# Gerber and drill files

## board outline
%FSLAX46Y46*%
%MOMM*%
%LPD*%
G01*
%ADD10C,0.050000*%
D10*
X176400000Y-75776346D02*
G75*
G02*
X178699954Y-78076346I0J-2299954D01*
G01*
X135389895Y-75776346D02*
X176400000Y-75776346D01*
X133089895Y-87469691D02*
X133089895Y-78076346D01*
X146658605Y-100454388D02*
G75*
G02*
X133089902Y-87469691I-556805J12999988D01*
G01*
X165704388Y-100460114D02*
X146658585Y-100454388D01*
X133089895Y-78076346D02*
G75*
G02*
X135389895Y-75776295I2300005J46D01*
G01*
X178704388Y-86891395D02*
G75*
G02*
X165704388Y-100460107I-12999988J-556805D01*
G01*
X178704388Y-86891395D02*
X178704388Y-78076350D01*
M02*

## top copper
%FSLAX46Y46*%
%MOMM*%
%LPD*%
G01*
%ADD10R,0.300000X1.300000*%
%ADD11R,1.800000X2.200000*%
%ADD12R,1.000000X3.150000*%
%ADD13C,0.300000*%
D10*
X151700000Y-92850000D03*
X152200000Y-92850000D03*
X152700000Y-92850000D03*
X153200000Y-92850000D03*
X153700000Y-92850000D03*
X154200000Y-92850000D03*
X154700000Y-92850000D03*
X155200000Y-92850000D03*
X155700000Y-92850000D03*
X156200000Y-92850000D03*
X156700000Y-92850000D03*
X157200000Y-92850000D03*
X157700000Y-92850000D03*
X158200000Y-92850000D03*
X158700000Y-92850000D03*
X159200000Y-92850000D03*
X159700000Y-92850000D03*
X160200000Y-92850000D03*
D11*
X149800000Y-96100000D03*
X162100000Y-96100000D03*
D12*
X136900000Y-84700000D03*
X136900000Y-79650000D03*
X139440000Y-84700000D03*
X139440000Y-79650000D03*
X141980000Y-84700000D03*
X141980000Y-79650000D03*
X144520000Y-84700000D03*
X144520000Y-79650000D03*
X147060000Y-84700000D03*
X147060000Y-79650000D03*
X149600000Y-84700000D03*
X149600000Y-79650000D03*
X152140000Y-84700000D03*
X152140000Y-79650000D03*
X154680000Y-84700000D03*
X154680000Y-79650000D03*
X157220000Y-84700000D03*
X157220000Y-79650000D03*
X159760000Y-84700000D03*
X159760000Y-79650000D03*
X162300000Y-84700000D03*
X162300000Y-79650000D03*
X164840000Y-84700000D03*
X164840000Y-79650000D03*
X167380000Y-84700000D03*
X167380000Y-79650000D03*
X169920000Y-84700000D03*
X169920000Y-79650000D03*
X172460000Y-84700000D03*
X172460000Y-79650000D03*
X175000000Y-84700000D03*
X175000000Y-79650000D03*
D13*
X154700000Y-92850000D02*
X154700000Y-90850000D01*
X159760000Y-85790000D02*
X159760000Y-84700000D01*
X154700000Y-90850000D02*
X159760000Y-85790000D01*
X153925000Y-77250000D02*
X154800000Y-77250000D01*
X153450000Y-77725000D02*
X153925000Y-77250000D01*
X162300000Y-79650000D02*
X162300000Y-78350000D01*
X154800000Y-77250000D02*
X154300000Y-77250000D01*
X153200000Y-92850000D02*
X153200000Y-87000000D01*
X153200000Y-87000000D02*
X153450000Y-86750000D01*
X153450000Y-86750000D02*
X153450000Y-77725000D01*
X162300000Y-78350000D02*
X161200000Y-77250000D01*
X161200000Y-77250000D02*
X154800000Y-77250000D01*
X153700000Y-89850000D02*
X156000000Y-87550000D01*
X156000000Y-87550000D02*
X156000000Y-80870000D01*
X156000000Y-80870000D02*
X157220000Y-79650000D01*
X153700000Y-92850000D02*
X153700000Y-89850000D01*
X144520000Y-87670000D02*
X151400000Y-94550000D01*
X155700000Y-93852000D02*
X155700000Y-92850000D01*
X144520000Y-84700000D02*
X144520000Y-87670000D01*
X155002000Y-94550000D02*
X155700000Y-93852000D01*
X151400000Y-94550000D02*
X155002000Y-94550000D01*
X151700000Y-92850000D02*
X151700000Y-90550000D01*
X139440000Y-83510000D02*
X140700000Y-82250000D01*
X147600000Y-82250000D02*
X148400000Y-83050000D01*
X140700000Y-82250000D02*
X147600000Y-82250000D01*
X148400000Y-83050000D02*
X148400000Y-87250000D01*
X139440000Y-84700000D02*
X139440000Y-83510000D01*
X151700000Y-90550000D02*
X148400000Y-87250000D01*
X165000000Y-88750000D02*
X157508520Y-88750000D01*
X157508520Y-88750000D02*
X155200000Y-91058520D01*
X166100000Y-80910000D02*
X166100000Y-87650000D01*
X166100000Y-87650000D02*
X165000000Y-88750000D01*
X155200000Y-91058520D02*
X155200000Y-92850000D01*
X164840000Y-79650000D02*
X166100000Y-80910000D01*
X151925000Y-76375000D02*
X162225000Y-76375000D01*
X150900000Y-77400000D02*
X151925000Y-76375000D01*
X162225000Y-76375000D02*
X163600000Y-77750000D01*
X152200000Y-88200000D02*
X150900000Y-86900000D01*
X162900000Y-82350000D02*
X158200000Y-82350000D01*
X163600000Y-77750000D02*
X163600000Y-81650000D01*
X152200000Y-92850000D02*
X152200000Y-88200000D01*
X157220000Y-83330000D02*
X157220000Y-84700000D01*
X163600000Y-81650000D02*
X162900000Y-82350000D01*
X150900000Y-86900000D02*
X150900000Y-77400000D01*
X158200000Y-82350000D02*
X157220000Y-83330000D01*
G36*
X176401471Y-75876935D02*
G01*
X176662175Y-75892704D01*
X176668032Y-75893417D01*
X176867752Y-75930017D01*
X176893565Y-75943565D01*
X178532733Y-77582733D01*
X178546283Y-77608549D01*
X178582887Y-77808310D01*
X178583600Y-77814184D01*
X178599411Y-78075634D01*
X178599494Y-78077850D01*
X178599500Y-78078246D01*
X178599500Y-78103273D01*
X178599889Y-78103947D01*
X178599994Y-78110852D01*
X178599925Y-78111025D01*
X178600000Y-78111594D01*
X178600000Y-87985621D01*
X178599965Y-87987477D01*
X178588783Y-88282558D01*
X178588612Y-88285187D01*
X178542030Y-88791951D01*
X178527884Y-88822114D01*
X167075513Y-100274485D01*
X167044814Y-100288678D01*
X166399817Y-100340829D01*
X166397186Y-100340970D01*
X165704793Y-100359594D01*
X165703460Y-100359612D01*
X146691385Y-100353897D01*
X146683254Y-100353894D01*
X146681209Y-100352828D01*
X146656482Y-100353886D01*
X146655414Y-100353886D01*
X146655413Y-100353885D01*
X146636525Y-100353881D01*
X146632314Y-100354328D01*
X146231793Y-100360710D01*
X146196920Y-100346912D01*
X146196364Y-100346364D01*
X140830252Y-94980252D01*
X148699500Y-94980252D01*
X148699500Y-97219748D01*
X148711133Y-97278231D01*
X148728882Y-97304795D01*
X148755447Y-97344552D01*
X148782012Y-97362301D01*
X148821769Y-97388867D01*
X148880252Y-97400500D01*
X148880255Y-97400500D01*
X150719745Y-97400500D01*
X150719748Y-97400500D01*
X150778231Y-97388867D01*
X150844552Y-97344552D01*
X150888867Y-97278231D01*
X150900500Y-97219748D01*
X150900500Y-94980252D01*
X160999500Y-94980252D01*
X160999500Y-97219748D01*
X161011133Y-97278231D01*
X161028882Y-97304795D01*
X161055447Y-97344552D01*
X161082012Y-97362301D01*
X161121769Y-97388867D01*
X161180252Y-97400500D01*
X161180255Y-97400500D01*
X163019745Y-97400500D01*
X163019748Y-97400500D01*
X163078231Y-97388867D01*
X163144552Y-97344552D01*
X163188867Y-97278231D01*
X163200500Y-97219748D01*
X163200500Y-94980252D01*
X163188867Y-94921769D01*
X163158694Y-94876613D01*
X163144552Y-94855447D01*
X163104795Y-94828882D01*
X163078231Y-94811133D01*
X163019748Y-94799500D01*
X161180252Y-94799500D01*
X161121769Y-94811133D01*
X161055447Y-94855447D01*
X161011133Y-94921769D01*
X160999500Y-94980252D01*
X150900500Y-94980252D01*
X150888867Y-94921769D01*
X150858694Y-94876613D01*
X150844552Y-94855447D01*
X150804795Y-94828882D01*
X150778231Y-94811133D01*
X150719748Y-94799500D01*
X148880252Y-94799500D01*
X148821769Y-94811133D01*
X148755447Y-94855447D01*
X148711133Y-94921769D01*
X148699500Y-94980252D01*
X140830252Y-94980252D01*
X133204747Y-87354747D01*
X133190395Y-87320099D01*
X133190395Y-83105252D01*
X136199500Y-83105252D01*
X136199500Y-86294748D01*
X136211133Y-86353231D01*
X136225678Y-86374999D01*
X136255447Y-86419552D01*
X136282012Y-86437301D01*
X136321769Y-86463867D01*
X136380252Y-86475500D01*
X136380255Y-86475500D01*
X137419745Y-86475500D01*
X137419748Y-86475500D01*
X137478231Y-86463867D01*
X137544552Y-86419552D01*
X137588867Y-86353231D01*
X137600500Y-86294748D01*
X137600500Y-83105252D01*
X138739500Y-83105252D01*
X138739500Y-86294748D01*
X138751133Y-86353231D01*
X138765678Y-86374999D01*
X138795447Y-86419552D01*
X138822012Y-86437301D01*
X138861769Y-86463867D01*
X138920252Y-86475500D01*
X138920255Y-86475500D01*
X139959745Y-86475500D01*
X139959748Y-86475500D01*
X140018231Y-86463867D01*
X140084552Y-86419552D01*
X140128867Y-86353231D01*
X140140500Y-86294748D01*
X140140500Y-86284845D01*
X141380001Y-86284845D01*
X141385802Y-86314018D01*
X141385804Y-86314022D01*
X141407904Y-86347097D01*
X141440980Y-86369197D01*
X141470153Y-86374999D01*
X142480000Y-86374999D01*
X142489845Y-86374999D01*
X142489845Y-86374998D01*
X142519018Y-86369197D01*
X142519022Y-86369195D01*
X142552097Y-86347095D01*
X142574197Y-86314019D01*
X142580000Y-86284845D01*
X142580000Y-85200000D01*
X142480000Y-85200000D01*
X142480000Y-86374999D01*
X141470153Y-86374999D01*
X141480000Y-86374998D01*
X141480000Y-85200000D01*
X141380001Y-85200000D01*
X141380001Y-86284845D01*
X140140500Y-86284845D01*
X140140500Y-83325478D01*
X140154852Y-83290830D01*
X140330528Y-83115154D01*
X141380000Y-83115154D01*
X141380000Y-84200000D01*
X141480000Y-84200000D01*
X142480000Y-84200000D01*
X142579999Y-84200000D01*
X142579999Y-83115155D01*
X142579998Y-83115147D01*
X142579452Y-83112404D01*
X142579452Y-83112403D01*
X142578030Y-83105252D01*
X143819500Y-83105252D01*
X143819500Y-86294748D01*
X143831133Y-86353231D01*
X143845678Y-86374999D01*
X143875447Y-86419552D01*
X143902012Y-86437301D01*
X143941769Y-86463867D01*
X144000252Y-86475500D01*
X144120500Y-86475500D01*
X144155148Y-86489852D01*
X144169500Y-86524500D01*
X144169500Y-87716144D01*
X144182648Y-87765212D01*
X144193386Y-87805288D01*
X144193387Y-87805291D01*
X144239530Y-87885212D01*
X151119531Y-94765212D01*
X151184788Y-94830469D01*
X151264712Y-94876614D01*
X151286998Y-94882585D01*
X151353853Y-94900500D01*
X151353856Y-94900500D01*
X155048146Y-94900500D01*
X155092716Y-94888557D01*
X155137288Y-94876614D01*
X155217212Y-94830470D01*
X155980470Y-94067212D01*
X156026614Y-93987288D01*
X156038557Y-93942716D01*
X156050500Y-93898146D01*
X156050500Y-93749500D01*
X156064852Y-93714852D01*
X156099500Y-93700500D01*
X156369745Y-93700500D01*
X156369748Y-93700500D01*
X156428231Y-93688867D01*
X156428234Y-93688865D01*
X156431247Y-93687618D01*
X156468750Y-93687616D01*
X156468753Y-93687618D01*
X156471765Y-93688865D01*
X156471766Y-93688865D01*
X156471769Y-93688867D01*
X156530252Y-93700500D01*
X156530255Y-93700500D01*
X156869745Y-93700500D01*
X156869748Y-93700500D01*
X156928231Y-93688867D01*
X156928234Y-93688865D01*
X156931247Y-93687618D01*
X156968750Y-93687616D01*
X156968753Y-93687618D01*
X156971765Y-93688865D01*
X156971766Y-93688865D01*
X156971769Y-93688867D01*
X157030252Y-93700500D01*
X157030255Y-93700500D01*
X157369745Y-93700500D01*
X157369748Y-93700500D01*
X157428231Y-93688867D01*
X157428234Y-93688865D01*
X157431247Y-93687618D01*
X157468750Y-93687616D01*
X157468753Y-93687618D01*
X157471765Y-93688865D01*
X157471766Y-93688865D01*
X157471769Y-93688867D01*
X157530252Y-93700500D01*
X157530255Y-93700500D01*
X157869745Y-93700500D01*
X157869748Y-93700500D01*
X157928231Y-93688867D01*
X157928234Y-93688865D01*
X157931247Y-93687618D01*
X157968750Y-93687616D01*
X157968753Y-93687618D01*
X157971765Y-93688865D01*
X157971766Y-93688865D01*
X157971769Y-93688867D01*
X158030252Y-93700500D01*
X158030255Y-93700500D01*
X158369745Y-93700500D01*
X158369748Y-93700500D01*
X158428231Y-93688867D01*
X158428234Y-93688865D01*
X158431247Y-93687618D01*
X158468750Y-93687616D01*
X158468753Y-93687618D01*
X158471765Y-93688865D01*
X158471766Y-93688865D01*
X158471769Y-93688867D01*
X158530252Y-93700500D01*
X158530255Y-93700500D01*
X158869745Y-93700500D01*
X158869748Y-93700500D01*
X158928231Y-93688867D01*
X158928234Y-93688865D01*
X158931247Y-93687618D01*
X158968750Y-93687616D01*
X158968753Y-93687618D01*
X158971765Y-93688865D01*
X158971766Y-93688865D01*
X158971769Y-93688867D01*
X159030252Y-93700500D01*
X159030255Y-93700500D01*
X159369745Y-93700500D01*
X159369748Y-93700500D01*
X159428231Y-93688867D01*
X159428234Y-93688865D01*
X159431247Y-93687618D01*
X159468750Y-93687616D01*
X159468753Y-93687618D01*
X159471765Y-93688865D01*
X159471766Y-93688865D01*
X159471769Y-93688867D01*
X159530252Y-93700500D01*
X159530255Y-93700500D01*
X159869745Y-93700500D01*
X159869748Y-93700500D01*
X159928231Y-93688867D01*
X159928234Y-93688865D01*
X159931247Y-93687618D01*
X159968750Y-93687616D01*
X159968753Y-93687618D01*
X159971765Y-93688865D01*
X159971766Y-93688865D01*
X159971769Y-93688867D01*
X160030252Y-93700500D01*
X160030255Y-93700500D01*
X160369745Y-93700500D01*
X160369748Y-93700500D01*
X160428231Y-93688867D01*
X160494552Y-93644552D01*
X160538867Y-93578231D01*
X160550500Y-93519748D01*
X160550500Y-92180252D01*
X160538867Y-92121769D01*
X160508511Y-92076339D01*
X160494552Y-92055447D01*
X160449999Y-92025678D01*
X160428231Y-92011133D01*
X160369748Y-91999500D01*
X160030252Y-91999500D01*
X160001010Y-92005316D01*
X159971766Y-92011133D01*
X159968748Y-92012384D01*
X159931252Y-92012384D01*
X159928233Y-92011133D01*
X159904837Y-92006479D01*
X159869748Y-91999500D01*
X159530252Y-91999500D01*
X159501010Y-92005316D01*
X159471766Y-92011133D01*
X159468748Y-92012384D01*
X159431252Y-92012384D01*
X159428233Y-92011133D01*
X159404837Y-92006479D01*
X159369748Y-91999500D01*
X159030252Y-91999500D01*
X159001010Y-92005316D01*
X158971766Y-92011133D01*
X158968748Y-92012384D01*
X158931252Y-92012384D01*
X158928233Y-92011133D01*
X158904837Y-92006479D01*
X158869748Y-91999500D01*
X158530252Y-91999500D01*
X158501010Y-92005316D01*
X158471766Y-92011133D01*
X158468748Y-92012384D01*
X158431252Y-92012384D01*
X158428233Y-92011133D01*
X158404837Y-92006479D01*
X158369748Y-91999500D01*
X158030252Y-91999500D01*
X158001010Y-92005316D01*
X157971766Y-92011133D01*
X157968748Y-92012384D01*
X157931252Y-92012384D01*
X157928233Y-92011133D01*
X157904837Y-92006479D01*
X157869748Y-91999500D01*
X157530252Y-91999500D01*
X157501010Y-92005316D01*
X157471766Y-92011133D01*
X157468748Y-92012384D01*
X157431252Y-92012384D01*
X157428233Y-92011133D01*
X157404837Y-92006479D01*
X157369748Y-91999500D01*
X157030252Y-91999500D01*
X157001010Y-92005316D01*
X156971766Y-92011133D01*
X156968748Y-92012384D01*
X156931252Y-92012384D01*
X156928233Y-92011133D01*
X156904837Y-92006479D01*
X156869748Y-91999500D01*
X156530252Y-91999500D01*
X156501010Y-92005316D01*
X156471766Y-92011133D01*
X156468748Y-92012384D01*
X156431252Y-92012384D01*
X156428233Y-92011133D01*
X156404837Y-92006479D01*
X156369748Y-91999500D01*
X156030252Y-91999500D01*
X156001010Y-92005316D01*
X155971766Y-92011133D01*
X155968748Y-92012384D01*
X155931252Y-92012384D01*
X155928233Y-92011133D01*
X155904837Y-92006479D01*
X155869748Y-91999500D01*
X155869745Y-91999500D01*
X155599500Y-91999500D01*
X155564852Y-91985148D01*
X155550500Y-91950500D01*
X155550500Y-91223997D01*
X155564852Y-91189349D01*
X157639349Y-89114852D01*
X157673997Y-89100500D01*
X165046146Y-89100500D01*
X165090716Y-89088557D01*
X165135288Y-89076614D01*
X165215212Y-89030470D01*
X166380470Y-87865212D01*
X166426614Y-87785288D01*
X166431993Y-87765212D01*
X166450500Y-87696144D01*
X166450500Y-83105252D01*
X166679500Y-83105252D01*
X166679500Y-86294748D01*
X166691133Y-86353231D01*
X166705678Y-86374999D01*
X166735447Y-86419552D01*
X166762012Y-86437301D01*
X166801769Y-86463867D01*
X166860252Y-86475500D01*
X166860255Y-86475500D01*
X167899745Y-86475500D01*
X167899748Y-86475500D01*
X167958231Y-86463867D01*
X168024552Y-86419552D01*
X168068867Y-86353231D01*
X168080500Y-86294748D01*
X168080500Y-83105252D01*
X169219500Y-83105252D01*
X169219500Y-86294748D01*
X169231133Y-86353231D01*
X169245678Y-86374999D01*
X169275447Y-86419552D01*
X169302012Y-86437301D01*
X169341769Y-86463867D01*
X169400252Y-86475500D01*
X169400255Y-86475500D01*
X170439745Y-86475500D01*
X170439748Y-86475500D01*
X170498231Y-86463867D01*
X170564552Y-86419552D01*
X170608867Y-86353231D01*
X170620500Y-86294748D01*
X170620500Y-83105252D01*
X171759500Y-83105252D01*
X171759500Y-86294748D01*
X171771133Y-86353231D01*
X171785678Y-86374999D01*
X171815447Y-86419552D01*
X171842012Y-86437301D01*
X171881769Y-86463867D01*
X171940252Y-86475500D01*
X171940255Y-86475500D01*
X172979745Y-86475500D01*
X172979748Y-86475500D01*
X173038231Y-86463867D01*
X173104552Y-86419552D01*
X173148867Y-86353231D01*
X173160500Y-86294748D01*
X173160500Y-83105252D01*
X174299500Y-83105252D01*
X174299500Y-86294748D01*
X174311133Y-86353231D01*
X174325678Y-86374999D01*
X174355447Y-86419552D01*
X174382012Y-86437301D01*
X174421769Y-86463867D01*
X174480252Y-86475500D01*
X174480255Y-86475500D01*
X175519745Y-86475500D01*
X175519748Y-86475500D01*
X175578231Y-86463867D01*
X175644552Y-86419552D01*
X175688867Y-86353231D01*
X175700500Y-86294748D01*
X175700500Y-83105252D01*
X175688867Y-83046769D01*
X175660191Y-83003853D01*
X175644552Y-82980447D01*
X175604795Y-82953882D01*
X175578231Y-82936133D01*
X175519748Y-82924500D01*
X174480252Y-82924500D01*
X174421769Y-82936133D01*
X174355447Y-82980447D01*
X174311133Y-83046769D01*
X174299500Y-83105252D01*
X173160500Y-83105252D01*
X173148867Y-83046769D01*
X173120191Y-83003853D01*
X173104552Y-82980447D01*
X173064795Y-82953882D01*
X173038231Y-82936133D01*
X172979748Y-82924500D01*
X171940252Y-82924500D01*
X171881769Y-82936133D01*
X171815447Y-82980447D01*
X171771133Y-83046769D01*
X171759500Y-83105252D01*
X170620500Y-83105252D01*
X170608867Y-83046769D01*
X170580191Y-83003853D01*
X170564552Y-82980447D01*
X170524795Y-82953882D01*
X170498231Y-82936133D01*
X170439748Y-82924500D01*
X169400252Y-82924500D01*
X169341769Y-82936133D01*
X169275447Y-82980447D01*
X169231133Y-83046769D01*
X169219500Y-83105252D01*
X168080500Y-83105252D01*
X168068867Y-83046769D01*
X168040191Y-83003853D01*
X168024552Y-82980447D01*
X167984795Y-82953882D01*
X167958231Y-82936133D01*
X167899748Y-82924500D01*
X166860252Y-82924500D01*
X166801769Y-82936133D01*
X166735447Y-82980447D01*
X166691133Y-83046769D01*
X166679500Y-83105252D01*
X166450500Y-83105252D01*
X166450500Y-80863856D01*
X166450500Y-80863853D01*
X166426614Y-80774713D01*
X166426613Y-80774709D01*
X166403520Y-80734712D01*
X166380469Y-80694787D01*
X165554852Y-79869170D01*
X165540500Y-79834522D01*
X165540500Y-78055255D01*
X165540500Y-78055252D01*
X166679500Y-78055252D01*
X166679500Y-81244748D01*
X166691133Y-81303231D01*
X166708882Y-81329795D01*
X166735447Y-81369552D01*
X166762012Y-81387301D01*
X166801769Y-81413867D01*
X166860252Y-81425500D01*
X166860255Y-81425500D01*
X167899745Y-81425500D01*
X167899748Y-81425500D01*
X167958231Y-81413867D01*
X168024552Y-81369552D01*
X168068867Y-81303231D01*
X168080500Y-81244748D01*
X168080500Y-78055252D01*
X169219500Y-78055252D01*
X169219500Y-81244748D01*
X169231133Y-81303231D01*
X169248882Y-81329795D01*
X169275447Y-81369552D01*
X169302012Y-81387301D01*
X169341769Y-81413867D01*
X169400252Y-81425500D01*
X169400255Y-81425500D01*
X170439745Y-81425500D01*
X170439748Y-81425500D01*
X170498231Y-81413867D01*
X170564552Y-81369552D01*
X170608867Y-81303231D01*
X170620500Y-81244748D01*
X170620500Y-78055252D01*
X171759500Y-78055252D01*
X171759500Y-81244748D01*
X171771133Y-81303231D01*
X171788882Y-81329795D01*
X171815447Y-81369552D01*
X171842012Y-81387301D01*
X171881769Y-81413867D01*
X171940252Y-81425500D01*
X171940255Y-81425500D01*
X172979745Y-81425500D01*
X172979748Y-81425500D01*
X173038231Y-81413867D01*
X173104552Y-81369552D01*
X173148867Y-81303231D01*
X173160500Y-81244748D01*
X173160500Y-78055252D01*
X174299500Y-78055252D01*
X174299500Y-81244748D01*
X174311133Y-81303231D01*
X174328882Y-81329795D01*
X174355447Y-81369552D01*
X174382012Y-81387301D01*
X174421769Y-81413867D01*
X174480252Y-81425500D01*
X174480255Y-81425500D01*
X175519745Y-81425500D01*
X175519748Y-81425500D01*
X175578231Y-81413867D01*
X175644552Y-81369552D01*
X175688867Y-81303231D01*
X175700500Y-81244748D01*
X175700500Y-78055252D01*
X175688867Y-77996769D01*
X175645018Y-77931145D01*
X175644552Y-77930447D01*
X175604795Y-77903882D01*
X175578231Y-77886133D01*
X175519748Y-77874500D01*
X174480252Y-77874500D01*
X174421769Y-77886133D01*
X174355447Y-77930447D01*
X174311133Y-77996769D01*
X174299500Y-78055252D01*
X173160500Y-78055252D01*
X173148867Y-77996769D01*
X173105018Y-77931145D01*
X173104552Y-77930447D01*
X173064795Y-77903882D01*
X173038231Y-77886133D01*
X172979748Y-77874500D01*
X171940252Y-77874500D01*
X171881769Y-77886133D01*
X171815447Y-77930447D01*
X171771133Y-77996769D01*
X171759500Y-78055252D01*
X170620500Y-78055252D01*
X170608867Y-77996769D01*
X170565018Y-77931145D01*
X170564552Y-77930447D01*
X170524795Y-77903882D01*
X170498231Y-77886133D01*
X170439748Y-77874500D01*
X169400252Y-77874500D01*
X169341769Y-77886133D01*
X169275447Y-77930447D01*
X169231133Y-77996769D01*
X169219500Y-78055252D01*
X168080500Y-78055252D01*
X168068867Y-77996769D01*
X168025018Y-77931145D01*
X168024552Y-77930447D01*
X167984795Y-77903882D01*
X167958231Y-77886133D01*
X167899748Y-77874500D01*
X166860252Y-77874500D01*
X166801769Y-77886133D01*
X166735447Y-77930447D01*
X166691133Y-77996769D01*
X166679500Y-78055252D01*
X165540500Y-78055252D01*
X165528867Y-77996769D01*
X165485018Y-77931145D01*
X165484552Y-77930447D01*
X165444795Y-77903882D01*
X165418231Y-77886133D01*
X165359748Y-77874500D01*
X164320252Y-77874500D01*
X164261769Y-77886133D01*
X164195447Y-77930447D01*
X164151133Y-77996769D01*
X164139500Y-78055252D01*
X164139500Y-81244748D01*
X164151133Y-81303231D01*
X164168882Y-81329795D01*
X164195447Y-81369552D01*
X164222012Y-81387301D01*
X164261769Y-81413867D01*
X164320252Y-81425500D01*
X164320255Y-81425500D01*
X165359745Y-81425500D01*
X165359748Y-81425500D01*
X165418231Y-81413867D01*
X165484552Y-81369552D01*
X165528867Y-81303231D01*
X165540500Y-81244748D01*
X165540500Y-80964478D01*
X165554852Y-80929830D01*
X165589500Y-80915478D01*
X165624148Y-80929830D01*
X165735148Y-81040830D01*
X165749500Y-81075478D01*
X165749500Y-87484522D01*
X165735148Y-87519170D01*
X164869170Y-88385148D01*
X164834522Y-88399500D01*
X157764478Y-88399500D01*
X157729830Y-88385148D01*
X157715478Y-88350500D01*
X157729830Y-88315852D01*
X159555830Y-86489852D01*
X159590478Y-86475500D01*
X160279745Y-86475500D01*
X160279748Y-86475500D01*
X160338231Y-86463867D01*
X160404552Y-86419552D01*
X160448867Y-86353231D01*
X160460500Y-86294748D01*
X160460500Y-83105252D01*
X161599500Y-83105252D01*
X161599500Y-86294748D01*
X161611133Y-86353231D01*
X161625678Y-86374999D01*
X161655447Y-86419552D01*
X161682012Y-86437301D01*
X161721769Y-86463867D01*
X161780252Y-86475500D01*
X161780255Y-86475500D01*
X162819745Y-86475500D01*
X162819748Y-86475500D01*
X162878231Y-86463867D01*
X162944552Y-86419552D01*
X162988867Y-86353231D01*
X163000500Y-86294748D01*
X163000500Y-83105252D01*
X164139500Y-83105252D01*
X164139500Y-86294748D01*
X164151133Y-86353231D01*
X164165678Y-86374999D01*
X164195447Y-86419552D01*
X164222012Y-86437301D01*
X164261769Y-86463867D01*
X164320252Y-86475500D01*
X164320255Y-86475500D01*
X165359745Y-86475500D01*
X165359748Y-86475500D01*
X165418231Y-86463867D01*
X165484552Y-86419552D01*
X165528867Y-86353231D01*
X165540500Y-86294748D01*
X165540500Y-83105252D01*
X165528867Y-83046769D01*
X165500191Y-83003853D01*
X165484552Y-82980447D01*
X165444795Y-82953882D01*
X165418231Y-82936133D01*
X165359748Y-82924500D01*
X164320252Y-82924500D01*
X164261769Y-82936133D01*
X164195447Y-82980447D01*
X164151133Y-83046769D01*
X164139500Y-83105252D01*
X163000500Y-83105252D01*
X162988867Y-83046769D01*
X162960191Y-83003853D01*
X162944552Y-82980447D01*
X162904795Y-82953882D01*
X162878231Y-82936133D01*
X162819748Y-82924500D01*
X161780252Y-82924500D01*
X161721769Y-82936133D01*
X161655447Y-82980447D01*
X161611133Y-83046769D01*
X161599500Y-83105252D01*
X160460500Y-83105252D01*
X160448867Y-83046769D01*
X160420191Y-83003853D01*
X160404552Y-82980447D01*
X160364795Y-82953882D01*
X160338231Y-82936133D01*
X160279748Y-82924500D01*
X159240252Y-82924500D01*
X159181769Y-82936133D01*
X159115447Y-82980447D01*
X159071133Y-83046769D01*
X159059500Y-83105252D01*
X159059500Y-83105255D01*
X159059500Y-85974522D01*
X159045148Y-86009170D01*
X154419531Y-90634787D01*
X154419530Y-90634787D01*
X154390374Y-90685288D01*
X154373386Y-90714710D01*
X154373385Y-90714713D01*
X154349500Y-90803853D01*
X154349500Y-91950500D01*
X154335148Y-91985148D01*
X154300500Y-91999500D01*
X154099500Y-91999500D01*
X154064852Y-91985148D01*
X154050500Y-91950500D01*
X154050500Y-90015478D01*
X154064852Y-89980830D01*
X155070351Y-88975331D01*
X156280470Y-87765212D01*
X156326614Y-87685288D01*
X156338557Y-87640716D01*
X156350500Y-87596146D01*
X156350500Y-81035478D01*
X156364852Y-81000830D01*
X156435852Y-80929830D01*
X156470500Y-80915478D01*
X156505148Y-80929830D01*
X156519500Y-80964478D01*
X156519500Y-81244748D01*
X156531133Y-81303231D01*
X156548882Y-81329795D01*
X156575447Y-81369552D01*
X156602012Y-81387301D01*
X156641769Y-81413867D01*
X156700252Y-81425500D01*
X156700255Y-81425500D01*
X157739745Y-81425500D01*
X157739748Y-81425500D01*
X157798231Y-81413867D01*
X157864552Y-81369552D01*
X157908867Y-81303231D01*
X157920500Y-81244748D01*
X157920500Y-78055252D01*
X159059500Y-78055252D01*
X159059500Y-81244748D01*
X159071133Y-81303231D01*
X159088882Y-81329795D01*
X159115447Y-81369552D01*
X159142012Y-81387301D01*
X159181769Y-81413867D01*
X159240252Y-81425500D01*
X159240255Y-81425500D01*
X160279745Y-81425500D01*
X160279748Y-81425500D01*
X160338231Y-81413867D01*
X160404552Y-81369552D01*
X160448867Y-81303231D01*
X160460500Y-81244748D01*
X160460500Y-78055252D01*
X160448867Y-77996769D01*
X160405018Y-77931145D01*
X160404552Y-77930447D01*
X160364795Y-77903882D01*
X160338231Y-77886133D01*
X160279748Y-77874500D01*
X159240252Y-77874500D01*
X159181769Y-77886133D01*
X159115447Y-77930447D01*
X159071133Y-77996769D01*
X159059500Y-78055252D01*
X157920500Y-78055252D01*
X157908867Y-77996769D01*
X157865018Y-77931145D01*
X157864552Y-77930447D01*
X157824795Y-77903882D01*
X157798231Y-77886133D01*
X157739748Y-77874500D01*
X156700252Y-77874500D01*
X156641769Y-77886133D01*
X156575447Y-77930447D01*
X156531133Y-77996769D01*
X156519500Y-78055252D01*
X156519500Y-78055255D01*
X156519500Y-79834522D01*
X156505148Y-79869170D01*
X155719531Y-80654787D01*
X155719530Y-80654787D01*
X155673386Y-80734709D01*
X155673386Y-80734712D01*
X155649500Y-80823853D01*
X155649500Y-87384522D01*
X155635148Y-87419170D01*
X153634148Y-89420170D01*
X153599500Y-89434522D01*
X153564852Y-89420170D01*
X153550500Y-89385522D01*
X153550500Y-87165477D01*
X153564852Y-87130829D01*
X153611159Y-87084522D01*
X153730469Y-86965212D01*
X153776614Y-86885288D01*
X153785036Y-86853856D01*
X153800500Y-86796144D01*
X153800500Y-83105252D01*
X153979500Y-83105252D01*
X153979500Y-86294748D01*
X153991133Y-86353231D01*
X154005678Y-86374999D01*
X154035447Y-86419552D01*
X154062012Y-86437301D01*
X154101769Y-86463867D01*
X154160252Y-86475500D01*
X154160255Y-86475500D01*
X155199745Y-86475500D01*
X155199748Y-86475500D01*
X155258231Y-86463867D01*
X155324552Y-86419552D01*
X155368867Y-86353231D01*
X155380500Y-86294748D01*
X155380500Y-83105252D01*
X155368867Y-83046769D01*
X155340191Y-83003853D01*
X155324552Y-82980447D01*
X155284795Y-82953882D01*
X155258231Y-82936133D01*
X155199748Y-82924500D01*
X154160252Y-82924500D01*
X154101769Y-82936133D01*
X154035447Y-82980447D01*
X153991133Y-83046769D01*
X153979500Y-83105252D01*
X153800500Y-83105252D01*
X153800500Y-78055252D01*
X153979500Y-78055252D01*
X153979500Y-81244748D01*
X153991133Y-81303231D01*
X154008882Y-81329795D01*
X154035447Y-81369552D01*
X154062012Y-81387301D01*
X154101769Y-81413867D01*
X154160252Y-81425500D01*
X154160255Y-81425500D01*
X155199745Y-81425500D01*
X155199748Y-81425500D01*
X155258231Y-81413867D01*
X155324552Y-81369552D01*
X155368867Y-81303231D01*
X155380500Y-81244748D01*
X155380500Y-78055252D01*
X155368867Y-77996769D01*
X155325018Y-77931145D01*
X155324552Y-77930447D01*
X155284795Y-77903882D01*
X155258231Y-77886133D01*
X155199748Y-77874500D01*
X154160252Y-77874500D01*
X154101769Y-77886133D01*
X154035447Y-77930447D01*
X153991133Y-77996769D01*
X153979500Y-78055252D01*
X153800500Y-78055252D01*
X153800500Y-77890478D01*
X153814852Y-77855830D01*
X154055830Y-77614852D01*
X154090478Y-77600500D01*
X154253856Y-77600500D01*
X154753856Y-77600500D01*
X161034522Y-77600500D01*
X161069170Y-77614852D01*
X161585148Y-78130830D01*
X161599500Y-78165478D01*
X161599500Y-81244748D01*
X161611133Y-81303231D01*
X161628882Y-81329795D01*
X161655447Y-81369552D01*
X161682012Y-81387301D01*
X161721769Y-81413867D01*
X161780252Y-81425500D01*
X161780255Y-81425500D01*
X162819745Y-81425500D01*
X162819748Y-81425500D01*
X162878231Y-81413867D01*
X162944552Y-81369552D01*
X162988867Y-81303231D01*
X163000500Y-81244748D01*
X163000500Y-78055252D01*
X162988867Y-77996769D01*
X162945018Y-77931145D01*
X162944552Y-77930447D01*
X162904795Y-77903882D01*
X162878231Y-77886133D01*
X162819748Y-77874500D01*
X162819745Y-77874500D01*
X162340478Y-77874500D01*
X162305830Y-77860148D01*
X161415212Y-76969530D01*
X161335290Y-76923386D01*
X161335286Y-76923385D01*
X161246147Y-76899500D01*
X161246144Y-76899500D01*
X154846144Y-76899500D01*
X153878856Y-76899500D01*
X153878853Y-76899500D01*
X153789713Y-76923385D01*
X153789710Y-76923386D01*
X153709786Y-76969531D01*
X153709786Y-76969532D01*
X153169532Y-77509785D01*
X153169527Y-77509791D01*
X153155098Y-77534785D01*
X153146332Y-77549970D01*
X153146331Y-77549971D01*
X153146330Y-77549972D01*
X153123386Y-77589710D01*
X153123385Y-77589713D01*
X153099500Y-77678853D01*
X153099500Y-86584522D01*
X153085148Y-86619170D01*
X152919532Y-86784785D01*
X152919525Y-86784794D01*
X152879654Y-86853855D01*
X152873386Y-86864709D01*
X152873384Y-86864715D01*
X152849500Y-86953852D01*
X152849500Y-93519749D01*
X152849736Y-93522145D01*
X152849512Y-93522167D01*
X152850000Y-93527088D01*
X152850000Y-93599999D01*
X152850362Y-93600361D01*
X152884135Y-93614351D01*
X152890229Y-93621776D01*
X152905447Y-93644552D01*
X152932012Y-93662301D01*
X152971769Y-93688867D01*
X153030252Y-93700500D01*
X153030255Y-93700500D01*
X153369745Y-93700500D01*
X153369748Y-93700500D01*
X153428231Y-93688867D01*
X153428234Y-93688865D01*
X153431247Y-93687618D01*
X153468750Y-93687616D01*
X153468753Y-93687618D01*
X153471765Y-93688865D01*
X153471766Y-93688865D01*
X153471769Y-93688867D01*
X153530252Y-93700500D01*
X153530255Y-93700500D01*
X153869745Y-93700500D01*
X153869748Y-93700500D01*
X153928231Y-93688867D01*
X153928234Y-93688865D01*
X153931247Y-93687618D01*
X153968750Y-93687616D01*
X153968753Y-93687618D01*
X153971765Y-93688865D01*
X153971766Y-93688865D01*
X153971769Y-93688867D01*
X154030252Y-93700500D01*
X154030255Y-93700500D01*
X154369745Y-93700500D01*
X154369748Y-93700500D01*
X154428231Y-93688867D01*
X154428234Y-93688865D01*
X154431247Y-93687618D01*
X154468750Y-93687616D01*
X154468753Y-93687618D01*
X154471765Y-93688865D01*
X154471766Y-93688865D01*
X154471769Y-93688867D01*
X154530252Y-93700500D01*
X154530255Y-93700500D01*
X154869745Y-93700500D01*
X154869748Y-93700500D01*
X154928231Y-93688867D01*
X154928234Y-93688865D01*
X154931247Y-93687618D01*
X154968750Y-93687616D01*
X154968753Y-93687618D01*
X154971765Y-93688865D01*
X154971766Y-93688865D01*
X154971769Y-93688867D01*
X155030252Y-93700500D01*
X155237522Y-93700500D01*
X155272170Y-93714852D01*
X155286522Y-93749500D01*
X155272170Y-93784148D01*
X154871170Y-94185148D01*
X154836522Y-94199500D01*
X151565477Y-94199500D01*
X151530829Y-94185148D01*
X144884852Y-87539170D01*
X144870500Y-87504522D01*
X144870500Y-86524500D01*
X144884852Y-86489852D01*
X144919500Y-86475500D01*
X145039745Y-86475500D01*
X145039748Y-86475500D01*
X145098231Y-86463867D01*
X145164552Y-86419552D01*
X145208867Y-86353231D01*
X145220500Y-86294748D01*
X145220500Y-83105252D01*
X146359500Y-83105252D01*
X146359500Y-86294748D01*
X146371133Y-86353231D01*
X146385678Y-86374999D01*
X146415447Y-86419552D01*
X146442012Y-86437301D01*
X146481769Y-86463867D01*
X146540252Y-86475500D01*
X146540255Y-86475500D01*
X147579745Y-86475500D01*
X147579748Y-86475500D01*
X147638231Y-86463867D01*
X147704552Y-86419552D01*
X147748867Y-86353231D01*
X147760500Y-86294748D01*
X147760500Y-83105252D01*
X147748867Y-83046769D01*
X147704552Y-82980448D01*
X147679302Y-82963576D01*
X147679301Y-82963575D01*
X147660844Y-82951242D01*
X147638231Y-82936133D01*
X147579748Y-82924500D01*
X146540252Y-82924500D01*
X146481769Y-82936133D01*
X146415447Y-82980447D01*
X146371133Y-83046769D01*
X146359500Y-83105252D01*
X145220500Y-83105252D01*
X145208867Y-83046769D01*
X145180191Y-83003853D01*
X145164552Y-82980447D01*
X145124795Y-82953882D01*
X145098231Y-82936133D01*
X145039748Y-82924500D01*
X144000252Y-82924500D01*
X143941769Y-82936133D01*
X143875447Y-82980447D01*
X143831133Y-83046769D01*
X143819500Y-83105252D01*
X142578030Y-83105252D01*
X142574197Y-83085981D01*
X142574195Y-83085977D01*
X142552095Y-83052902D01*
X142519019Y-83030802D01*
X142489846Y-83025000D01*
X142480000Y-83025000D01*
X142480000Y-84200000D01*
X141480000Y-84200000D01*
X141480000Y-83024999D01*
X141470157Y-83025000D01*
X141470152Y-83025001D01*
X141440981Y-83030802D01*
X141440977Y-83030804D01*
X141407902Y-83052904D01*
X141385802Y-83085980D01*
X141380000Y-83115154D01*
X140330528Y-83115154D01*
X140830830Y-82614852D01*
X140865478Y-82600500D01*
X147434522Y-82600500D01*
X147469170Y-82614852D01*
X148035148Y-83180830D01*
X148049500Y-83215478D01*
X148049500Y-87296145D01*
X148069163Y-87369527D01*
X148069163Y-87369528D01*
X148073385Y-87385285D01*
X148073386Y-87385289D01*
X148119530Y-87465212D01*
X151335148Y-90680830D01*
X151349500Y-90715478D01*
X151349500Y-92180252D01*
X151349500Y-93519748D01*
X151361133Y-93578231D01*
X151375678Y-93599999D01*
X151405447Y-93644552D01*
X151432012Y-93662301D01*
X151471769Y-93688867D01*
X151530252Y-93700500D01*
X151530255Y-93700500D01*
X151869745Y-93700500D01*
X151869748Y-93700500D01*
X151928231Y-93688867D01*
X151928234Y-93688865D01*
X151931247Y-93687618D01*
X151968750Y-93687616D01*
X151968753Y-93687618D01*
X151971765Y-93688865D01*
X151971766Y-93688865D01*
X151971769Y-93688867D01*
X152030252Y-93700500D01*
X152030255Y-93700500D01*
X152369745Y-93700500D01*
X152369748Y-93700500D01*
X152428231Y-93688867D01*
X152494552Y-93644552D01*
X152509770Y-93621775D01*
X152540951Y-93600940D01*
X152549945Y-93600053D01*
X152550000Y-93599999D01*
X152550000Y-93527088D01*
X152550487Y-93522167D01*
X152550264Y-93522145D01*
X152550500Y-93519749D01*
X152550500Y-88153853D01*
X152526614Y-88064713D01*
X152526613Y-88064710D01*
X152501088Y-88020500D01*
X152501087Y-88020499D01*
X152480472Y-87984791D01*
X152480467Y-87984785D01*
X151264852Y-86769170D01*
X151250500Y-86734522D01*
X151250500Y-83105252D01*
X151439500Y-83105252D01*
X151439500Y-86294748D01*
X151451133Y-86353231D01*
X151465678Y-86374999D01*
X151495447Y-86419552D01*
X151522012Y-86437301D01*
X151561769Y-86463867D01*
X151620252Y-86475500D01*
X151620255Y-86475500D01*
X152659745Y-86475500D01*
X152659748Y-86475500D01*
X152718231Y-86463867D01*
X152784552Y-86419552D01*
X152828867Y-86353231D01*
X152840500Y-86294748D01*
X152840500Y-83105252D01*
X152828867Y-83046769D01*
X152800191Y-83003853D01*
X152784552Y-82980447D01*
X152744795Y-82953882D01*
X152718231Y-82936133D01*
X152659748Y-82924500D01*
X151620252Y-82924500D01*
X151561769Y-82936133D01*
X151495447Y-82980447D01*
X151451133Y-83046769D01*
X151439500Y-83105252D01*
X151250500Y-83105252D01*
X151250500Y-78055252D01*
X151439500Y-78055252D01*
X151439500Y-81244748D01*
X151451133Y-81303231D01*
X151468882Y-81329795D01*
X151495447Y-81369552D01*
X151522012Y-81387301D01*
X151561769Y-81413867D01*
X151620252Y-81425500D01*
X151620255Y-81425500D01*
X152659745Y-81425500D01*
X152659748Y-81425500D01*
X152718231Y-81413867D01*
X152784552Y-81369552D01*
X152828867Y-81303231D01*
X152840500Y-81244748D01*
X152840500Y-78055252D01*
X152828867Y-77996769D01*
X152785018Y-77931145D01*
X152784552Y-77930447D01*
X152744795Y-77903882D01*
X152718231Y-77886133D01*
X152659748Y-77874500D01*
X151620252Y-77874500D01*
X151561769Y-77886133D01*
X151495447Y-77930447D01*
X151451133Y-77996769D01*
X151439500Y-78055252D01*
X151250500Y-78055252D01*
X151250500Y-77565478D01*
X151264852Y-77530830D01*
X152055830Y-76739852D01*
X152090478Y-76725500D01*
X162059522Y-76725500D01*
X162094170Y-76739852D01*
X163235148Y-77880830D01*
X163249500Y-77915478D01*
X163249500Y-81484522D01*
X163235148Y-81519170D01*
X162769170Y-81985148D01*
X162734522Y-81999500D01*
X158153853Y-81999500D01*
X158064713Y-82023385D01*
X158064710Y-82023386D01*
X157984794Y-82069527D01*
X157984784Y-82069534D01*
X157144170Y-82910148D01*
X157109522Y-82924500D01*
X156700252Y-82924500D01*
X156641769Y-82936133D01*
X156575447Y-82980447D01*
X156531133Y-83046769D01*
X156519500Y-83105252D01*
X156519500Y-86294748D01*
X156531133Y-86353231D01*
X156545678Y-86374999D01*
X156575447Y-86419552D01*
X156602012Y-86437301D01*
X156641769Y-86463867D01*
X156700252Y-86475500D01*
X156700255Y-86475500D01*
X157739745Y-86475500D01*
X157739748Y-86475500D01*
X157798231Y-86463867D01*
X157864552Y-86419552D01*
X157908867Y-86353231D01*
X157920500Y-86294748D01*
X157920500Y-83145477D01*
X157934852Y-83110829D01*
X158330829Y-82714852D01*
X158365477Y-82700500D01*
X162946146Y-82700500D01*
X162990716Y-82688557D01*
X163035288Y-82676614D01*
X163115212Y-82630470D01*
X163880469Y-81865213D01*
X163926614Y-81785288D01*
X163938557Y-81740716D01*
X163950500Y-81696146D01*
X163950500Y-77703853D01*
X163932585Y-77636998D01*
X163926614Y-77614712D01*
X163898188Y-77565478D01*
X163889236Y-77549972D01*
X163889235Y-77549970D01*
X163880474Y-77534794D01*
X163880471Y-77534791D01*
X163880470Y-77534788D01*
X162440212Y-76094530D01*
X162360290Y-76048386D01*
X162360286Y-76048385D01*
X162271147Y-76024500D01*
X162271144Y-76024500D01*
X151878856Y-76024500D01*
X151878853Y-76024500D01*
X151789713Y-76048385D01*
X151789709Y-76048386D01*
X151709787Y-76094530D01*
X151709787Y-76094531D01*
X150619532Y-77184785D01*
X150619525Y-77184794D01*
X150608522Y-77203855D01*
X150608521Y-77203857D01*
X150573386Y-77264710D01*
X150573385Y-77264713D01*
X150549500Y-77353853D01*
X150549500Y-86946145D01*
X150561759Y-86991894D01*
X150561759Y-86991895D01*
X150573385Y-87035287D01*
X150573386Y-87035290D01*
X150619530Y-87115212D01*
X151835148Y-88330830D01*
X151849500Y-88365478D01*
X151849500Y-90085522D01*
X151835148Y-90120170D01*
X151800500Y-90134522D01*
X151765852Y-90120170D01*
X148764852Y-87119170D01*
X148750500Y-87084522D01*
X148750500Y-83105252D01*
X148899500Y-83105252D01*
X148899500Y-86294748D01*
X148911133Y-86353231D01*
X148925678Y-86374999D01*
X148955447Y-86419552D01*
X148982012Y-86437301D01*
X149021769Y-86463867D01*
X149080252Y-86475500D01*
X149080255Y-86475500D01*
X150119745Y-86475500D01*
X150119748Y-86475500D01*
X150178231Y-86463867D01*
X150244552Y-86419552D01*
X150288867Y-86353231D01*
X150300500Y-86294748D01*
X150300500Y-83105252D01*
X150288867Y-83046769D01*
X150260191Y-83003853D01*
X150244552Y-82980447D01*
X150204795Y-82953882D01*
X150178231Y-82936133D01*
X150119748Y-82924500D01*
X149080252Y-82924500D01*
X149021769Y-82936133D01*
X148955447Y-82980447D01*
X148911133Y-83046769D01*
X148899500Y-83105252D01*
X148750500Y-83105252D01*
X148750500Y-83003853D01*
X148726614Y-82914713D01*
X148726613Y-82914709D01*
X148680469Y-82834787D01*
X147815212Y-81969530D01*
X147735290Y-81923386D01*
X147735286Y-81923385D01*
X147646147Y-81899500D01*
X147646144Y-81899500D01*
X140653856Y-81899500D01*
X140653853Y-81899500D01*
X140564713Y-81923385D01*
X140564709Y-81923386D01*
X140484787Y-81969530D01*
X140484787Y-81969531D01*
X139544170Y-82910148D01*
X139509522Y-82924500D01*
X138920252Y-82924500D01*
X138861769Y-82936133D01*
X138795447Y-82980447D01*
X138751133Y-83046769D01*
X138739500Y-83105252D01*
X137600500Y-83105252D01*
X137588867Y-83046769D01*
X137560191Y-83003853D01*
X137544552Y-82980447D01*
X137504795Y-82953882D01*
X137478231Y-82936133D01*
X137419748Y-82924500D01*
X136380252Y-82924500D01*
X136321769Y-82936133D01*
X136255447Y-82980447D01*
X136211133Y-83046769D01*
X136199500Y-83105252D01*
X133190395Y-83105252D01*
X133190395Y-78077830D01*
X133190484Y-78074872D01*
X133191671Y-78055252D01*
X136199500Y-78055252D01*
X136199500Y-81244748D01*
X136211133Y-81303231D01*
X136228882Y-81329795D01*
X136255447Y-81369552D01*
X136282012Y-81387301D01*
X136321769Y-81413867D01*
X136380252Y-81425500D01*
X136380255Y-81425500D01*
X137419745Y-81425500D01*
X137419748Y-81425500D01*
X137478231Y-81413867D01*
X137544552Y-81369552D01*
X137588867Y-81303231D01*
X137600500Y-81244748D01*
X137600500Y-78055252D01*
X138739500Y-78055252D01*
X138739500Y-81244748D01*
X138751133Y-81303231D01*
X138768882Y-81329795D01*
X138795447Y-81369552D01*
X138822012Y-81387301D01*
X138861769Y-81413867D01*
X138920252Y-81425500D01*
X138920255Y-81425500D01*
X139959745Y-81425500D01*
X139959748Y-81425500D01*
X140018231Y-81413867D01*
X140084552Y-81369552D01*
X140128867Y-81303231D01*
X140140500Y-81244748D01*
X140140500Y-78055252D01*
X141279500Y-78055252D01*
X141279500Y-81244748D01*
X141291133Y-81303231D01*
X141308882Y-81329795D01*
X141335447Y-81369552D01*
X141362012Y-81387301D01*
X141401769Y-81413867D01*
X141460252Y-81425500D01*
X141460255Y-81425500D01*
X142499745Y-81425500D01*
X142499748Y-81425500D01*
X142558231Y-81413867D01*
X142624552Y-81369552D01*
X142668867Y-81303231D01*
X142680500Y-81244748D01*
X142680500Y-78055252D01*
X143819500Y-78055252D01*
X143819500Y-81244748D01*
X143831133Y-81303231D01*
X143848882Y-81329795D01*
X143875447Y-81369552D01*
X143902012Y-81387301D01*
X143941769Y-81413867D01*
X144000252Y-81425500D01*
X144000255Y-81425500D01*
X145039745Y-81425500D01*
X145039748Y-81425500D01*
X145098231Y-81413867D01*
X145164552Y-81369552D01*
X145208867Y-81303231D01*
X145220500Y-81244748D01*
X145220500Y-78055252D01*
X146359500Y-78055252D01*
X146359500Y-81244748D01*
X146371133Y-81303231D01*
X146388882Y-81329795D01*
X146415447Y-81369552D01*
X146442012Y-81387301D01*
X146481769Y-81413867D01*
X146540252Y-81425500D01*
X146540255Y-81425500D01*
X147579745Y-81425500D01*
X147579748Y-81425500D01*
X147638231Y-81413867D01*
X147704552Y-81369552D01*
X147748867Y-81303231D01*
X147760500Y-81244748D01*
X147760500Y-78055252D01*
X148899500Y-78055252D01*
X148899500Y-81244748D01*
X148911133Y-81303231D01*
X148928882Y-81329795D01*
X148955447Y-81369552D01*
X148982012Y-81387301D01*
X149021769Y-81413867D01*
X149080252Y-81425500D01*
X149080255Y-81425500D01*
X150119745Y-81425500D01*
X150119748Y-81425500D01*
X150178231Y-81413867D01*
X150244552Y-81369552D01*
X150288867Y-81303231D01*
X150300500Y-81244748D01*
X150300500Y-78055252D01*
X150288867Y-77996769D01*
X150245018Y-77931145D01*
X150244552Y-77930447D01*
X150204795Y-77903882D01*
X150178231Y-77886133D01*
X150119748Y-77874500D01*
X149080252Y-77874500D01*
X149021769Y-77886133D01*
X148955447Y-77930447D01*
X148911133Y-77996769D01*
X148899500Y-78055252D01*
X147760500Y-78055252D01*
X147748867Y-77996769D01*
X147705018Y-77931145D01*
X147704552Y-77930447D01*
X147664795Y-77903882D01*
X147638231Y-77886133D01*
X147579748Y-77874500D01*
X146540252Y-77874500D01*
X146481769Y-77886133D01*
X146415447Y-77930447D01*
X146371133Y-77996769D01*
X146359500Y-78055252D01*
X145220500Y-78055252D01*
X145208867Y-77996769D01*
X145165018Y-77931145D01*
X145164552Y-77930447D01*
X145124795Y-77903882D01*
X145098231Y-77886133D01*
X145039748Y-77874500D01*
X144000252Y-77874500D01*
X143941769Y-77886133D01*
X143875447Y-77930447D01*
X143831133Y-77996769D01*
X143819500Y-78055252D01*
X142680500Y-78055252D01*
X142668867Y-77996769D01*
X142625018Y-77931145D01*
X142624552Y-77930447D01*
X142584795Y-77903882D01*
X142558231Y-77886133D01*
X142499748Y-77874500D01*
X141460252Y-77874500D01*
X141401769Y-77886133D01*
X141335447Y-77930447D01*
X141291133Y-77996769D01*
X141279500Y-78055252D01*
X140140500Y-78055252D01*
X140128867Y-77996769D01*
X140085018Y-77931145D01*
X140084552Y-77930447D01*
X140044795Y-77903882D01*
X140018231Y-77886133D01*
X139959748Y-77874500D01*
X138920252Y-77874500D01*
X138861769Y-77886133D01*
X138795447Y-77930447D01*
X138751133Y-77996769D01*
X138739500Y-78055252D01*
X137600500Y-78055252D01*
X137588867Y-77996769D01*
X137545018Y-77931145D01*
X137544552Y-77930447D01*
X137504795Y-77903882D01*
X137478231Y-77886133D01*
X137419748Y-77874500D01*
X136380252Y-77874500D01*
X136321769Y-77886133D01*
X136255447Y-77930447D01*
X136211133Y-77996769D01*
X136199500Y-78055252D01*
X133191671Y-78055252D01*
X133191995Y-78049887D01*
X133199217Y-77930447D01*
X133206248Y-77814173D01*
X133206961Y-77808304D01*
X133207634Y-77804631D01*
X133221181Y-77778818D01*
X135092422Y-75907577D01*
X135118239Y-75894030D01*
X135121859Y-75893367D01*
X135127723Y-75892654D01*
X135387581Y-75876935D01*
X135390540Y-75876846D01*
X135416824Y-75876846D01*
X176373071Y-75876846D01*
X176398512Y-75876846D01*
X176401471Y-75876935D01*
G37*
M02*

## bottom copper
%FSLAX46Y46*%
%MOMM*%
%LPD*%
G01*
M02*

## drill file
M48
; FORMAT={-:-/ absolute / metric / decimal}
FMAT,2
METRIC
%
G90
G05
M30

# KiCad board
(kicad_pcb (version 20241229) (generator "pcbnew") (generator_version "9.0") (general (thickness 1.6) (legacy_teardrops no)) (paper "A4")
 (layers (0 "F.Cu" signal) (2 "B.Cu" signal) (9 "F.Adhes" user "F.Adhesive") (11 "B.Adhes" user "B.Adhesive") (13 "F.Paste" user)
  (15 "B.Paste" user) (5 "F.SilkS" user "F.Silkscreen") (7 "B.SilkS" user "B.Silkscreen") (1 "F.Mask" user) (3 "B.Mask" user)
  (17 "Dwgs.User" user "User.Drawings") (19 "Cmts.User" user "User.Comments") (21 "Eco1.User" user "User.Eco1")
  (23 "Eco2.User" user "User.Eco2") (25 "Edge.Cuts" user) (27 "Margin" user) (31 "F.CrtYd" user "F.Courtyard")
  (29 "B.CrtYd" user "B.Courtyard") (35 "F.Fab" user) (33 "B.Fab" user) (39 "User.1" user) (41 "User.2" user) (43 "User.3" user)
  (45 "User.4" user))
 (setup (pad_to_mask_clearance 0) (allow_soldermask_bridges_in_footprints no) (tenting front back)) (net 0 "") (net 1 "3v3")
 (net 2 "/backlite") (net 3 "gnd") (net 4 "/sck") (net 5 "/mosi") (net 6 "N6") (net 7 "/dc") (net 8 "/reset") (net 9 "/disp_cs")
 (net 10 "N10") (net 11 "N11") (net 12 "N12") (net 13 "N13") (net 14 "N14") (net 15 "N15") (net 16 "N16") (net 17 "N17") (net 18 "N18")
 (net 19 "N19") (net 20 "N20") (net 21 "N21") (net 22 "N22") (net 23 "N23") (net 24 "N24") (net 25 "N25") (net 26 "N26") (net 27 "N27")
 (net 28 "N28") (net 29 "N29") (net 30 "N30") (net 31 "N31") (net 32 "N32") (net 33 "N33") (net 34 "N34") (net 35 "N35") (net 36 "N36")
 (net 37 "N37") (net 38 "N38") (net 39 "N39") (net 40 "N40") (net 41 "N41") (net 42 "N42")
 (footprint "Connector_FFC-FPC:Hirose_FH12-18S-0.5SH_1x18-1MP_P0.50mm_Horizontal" (layer "F.Cu") (at 155.95 94.7)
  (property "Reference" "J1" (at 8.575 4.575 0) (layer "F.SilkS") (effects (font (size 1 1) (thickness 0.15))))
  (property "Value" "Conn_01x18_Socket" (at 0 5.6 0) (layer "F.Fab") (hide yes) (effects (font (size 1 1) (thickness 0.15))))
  (pad "1" smd rect (at -4.25 -1.85) (size 0.3 1.3) (layers "F.Cu" "F.Mask" "F.Paste") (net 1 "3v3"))
  (pad "2" smd rect (at -3.75 -1.85) (size 0.3 1.3) (layers "F.Cu" "F.Mask" "F.Paste") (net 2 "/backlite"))
  (pad "3" smd rect (at -3.25 -1.85) (size 0.3 1.3) (layers "F.Cu" "F.Mask" "F.Paste") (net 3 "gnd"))
  (pad "4" smd rect (at -2.75 -1.85) (size 0.3 1.3) (layers "F.Cu" "F.Mask" "F.Paste") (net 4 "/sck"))
  (pad "5" smd rect (at -2.25 -1.85) (size 0.3 1.3) (layers "F.Cu" "F.Mask" "F.Paste") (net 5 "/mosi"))
  (pad "6" smd rect (at -1.75 -1.85) (size 0.3 1.3) (layers "F.Cu" "F.Mask" "F.Paste") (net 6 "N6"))
  (pad "7" smd rect (at -1.25 -1.85) (size 0.3 1.3) (layers "F.Cu" "F.Mask" "F.Paste") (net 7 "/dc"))
  (pad "8" smd rect (at -0.75 -1.85) (size 0.3 1.3) (layers "F.Cu" "F.Mask" "F.Paste") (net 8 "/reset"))
  (pad "9" smd rect (at -0.25 -1.85) (size 0.3 1.3) (layers "F.Cu" "F.Mask" "F.Paste") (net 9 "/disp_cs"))
  (pad "10" smd rect (at 0.25 -1.85) (size 0.3 1.3) (layers "F.Cu" "F.Mask" "F.Paste") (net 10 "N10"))
  (pad "11" smd rect (at 0.75 -1.85) (size 0.3 1.3) (layers "F.Cu" "F.Mask" "F.Paste") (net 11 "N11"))
  (pad "12" smd rect (at 1.25 -1.85) (size 0.3 1.3) (layers "F.Cu" "F.Mask" "F.Paste") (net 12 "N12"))
  (pad "13" smd rect (at 1.75 -1.85) (size 0.3 1.3) (layers "F.Cu" "F.Mask" "F.Paste") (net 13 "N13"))
  (pad "14" smd rect (at 2.25 -1.85) (size 0.3 1.3) (layers "F.Cu" "F.Mask" "F.Paste") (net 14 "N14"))
  (pad "15" smd rect (at 2.75 -1.85) (size 0.3 1.3) (layers "F.Cu" "F.Mask" "F.Paste") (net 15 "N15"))
  (pad "16" smd rect (at 3.25 -1.85) (size 0.3 1.3) (layers "F.Cu" "F.Mask" "F.Paste") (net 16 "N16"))
  (pad "17" smd rect (at 3.75 -1.85) (size 0.3 1.3) (layers "F.Cu" "F.Mask" "F.Paste") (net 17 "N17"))
  (pad "18" smd rect (at 4.25 -1.85) (size 0.3 1.3) (layers "F.Cu" "F.Mask" "F.Paste") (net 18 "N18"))
  (pad "MP" smd rect (at -6.15 1.4) (size 1.8 2.2) (layers "F.Cu" "F.Mask" "F.Paste"))
  (pad "MP" smd rect (at 6.15 1.4) (size 1.8 2.2) (layers "F.Cu" "F.Mask" "F.Paste")))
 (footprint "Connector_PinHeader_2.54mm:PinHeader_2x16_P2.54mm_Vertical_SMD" (layer "F.Cu") (at 155.95 82.175 90)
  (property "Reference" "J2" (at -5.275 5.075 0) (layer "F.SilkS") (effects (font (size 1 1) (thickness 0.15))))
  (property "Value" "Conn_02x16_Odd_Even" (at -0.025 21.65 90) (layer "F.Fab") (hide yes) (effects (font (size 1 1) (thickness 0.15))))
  (pad "1" smd rect (at -2.525 -19.05 90) (size 3.15 1) (layers "F.Cu" "F.Mask" "F.Paste") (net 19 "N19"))
  (pad "2" smd rect (at 2.525 -19.05 90) (size 3.15 1) (layers "F.Cu" "F.Mask" "F.Paste") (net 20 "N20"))
  (pad "3" smd rect (at -2.525 -16.51 90) (size 3.15 1) (layers "F.Cu" "F.Mask" "F.Paste") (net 1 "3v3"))
  (pad "4" smd rect (at 2.525 -16.51 90) (size 3.15 1) (layers "F.Cu" "F.Mask" "F.Paste") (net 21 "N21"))
  (pad "5" smd rect (at -2.525 -13.97 90) (size 3.15 1) (layers "F.Cu" "F.Mask" "F.Paste") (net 3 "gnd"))
  (pad "6" smd rect (at 2.525 -13.97 90) (size 3.15 1) (layers "F.Cu" "F.Mask" "F.Paste") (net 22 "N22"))
  (pad "7" smd rect (at -2.525 -11.43 90) (size 3.15 1) (layers "F.Cu" "F.Mask" "F.Paste") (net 9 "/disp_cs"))
  (pad "8" smd rect (at 2.525 -11.43 90) (size 3.15 1) (layers "F.Cu" "F.Mask" "F.Paste") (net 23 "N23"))
  (pad "9" smd rect (at -2.525 -8.89 90) (size 3.15 1) (layers "F.Cu" "F.Mask" "F.Paste") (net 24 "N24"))
  (pad "10" smd rect (at 2.525 -8.89 90) (size 3.15 1) (layers "F.Cu" "F.Mask" "F.Paste") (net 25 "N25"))
  (pad "11" smd rect (at -2.525 -6.35 90) (size 3.15 1) (layers "F.Cu" "F.Mask" "F.Paste") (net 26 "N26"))
  (pad "12" smd rect (at 2.525 -6.35 90) (size 3.15 1) (layers "F.Cu" "F.Mask" "F.Paste") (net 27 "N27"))
  (pad "13" smd rect (at -2.525 -3.81 90) (size 3.15 1) (layers "F.Cu" "F.Mask" "F.Paste") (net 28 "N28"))
  (pad "14" smd rect (at 2.525 -3.81 90) (size 3.15 1) (layers "F.Cu" "F.Mask" "F.Paste") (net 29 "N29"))
  (pad "15" smd rect (at -2.525 -1.27 90) (size 3.15 1) (layers "F.Cu" "F.Mask" "F.Paste") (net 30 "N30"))
  (pad "16" smd rect (at 2.525 -1.27 90) (size 3.15 1) (layers "F.Cu" "F.Mask" "F.Paste") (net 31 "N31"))
  (pad "17" smd rect (at -2.525 1.27 90) (size 3.15 1) (layers "F.Cu" "F.Mask" "F.Paste") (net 2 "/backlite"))
  (pad "18" smd rect (at 2.525 1.27 90) (size 3.15 1) (layers "F.Cu" "F.Mask" "F.Paste") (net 5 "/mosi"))
  (pad "19" smd rect (at -2.525 3.81 90) (size 3.15 1) (layers "F.Cu" "F.Mask" "F.Paste") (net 7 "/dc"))
  (pad "20" smd rect (at 2.525 3.81 90) (size 3.15 1) (layers "F.Cu" "F.Mask" "F.Paste") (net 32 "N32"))
  (pad "21" smd rect (at -2.525 6.35 90) (size 3.15 1) (layers "F.Cu" "F.Mask" "F.Paste") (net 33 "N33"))
  (pad "22" smd rect (at 2.525 6.35 90) (size 3.15 1) (layers "F.Cu" "F.Mask" "F.Paste") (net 4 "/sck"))
  (pad "23" smd rect (at -2.525 8.89 90) (size 3.15 1) (layers "F.Cu" "F.Mask" "F.Paste") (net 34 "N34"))
  (pad "24" smd rect (at 2.525 8.89 90) (size 3.15 1) (layers "F.Cu" "F.Mask" "F.Paste") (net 8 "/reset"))
  (pad "25" smd rect (at -2.525 11.43 90) (size 3.15 1) (layers "F.Cu" "F.Mask" "F.Paste") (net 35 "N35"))
  (pad "26" smd rect (at 2.525 11.43 90) (size 3.15 1) (layers "F.Cu" "F.Mask" "F.Paste") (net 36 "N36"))
  (pad "27" smd rect (at -2.525 13.97 90) (size 3.15 1) (layers "F.Cu" "F.Mask" "F.Paste") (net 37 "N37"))
  (pad "28" smd rect (at 2.525 13.97 90) (size 3.15 1) (layers "F.Cu" "F.Mask" "F.Paste") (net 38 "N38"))
  (pad "29" smd rect (at -2.525 16.51 90) (size 3.15 1) (layers "F.Cu" "F.Mask" "F.Paste") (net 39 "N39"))
  (pad "30" smd rect (at 2.525 16.51 90) (size 3.15 1) (layers "F.Cu" "F.Mask" "F.Paste") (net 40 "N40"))
  (pad "31" smd rect (at -2.525 19.05 90) (size 3.15 1) (layers "F.Cu" "F.Mask" "F.Paste") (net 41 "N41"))
  (pad "32" smd rect (at 2.525 19.05 90) (size 3.15 1) (layers "F.Cu" "F.Mask" "F.Paste") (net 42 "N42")))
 (gr_arc (start 176.4 75.776346) (mid 178.026346 76.45) (end 178.7 78.076346) (stroke (width 0.05) (type default)) (layer "Edge.Cuts"))
 (gr_line (start 135.389895 75.776346) (end 176.4 75.776346) (stroke (width 0.05) (type default)) (layer "Edge.Cuts"))
 (gr_line (start 133.089895 87.469691) (end 133.089895 78.076346) (stroke (width 0.05) (type default)) (layer "Edge.Cuts"))
 (gr_arc (start 146.658605 100.454388) (mid 137.105527 96.855292) (end 133.089895 87.469691) (stroke (width 0.05) (type default))
  (layer "Edge.Cuts"))
 (gr_line (start 165.704388 100.460114) (end 146.658585 100.454388) (stroke (width 0.05) (type default)) (layer "Edge.Cuts"))
 (gr_arc (start 133.089895 78.076346) (mid 133.763549 76.45) (end 135.389895 75.776346) (stroke (width 0.05) (type default))
  (layer "Edge.Cuts"))
 (gr_arc (start 178.704388 86.891395) (mid 175.1 96.45) (end 165.704388 100.460114) (stroke (width 0.05) (type default)) (layer "Edge.Cuts"))
 (gr_line (start 178.704388 86.891395) (end 178.704388 78.07635) (stroke (width 0.05) (type default)) (layer "Edge.Cuts"))
 (segment (start 154.7 92.85) (end 154.7 90.85) (width 0.3) (layer "F.Cu") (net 7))
 (segment (start 159.76 85.79) (end 159.76 84.7) (width 0.3) (layer "F.Cu") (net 7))
 (segment (start 154.7 90.85) (end 159.76 85.79) (width 0.3) (layer "F.Cu") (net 7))
 (segment (start 153.925 77.25) (end 154.8 77.25) (width 0.3) (layer "F.Cu") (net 4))
 (segment (start 153.45 77.725) (end 153.925 77.25) (width 0.3) (layer "F.Cu") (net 4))
 (segment (start 162.3 79.65) (end 162.3 78.35) (width 0.3) (layer "F.Cu") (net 4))
 (segment (start 154.8 77.25) (end 154.3 77.25) (width 0.3) (layer "F.Cu") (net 4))
 (segment (start 153.2 92.85) (end 153.2 87) (width 0.3) (layer "F.Cu") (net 4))
 (segment (start 153.2 87) (end 153.45 86.75) (width 0.3) (layer "F.Cu") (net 4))
 (segment (start 153.45 86.75) (end 153.45 77.725) (width 0.3) (layer "F.Cu") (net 4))
 (segment (start 162.3 78.35) (end 161.2 77.25) (width 0.3) (layer "F.Cu") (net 4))
 (segment (start 161.2 77.25) (end 154.8 77.25) (width 0.3) (layer "F.Cu") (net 4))
 (segment (start 153.7 89.85) (end 156 87.55) (width 0.3) (layer "F.Cu") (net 5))
 (segment (start 156 87.55) (end 156 80.87) (width 0.3) (layer "F.Cu") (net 5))
 (segment (start 156 80.87) (end 157.22 79.65) (width 0.3) (layer "F.Cu") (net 5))
 (segment (start 153.7 92.85) (end 153.7 89.85) (width 0.3) (layer "F.Cu") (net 5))
 (segment (start 144.52 87.67) (end 151.4 94.55) (width 0.3) (layer "F.Cu") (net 9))
 (segment (start 155.7 93.852) (end 155.7 92.85) (width 0.3) (layer "F.Cu") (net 9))
 (segment (start 144.52 84.7) (end 144.52 87.67) (width 0.3) (layer "F.Cu") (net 9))
 (segment (start 155.002 94.55) (end 155.7 93.852) (width 0.3) (layer "F.Cu") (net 9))
 (segment (start 151.4 94.55) (end 155.002 94.55) (width 0.3) (layer "F.Cu") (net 9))
 (segment (start 151.7 92.85) (end 151.7 90.55) (width 0.3) (layer "F.Cu") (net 1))
 (segment (start 139.44 83.51) (end 140.7 82.25) (width 0.3) (layer "F.Cu") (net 1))
 (segment (start 147.6 82.25) (end 148.4 83.05) (width 0.3) (layer "F.Cu") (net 1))
 (segment (start 140.7 82.25) (end 147.6 82.25) (width 0.3) (layer "F.Cu") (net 1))
 (segment (start 148.4 83.05) (end 148.4 87.25) (width 0.3) (layer "F.Cu") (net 1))
 (segment (start 139.44 84.7) (end 139.44 83.51) (width 0.3) (layer "F.Cu") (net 1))
 (segment (start 151.7 90.55) (end 148.4 87.25) (width 0.3) (layer "F.Cu") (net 1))
 (segment (start 165 88.75) (end 157.50852 88.75) (width 0.3) (layer "F.Cu") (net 8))
 (segment (start 157.50852 88.75) (end 155.2 91.05852) (width 0.3) (layer "F.Cu") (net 8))
 (segment (start 166.1 80.91) (end 166.1 87.65) (width 0.3) (layer "F.Cu") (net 8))
 (segment (start 166.1 87.65) (end 165 88.75) (width 0.3) (layer "F.Cu") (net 8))
 (segment (start 155.2 91.05852) (end 155.2 92.85) (width 0.3) (layer "F.Cu") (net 8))
 (segment (start 164.84 79.65) (end 166.1 80.91) (width 0.3) (layer "F.Cu") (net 8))
 (segment (start 151.925 76.375) (end 162.225 76.375) (width 0.3) (layer "F.Cu") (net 2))
 (segment (start 150.9 77.4) (end 151.925 76.375) (width 0.3) (layer "F.Cu") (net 2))
 (segment (start 162.225 76.375) (end 163.6 77.75) (width 0.3) (layer "F.Cu") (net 2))
 (segment (start 152.2 88.2) (end 150.9 86.9) (width 0.3) (layer "F.Cu") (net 2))
 (segment (start 162.9 82.35) (end 158.2 82.35) (width 0.3) (layer "F.Cu") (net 2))
 (segment (start 163.6 77.75) (end 163.6 81.65) (width 0.3) (layer "F.Cu") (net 2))
 (segment (start 152.2 92.85) (end 152.2 88.2) (width 0.3) (layer "F.Cu") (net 2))
 (segment (start 157.22 83.33) (end 157.22 84.7) (width 0.3) (layer "F.Cu") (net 2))
 (segment (start 163.6 81.65) (end 162.9 82.35) (width 0.3) (layer "F.Cu") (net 2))
 (segment (start 150.9 86.9) (end 150.9 77.4) (width 0.3) (layer "F.Cu") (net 2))
 (segment (start 158.2 82.35) (end 157.22 83.33) (width 0.3) (layer "F.Cu") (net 2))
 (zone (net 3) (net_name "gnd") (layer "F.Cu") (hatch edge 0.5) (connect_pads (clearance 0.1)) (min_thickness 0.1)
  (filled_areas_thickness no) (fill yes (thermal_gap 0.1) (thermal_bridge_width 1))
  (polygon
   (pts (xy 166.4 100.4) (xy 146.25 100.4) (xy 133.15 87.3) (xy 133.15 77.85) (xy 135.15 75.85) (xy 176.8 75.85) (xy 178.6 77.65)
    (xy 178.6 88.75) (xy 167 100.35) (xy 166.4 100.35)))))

